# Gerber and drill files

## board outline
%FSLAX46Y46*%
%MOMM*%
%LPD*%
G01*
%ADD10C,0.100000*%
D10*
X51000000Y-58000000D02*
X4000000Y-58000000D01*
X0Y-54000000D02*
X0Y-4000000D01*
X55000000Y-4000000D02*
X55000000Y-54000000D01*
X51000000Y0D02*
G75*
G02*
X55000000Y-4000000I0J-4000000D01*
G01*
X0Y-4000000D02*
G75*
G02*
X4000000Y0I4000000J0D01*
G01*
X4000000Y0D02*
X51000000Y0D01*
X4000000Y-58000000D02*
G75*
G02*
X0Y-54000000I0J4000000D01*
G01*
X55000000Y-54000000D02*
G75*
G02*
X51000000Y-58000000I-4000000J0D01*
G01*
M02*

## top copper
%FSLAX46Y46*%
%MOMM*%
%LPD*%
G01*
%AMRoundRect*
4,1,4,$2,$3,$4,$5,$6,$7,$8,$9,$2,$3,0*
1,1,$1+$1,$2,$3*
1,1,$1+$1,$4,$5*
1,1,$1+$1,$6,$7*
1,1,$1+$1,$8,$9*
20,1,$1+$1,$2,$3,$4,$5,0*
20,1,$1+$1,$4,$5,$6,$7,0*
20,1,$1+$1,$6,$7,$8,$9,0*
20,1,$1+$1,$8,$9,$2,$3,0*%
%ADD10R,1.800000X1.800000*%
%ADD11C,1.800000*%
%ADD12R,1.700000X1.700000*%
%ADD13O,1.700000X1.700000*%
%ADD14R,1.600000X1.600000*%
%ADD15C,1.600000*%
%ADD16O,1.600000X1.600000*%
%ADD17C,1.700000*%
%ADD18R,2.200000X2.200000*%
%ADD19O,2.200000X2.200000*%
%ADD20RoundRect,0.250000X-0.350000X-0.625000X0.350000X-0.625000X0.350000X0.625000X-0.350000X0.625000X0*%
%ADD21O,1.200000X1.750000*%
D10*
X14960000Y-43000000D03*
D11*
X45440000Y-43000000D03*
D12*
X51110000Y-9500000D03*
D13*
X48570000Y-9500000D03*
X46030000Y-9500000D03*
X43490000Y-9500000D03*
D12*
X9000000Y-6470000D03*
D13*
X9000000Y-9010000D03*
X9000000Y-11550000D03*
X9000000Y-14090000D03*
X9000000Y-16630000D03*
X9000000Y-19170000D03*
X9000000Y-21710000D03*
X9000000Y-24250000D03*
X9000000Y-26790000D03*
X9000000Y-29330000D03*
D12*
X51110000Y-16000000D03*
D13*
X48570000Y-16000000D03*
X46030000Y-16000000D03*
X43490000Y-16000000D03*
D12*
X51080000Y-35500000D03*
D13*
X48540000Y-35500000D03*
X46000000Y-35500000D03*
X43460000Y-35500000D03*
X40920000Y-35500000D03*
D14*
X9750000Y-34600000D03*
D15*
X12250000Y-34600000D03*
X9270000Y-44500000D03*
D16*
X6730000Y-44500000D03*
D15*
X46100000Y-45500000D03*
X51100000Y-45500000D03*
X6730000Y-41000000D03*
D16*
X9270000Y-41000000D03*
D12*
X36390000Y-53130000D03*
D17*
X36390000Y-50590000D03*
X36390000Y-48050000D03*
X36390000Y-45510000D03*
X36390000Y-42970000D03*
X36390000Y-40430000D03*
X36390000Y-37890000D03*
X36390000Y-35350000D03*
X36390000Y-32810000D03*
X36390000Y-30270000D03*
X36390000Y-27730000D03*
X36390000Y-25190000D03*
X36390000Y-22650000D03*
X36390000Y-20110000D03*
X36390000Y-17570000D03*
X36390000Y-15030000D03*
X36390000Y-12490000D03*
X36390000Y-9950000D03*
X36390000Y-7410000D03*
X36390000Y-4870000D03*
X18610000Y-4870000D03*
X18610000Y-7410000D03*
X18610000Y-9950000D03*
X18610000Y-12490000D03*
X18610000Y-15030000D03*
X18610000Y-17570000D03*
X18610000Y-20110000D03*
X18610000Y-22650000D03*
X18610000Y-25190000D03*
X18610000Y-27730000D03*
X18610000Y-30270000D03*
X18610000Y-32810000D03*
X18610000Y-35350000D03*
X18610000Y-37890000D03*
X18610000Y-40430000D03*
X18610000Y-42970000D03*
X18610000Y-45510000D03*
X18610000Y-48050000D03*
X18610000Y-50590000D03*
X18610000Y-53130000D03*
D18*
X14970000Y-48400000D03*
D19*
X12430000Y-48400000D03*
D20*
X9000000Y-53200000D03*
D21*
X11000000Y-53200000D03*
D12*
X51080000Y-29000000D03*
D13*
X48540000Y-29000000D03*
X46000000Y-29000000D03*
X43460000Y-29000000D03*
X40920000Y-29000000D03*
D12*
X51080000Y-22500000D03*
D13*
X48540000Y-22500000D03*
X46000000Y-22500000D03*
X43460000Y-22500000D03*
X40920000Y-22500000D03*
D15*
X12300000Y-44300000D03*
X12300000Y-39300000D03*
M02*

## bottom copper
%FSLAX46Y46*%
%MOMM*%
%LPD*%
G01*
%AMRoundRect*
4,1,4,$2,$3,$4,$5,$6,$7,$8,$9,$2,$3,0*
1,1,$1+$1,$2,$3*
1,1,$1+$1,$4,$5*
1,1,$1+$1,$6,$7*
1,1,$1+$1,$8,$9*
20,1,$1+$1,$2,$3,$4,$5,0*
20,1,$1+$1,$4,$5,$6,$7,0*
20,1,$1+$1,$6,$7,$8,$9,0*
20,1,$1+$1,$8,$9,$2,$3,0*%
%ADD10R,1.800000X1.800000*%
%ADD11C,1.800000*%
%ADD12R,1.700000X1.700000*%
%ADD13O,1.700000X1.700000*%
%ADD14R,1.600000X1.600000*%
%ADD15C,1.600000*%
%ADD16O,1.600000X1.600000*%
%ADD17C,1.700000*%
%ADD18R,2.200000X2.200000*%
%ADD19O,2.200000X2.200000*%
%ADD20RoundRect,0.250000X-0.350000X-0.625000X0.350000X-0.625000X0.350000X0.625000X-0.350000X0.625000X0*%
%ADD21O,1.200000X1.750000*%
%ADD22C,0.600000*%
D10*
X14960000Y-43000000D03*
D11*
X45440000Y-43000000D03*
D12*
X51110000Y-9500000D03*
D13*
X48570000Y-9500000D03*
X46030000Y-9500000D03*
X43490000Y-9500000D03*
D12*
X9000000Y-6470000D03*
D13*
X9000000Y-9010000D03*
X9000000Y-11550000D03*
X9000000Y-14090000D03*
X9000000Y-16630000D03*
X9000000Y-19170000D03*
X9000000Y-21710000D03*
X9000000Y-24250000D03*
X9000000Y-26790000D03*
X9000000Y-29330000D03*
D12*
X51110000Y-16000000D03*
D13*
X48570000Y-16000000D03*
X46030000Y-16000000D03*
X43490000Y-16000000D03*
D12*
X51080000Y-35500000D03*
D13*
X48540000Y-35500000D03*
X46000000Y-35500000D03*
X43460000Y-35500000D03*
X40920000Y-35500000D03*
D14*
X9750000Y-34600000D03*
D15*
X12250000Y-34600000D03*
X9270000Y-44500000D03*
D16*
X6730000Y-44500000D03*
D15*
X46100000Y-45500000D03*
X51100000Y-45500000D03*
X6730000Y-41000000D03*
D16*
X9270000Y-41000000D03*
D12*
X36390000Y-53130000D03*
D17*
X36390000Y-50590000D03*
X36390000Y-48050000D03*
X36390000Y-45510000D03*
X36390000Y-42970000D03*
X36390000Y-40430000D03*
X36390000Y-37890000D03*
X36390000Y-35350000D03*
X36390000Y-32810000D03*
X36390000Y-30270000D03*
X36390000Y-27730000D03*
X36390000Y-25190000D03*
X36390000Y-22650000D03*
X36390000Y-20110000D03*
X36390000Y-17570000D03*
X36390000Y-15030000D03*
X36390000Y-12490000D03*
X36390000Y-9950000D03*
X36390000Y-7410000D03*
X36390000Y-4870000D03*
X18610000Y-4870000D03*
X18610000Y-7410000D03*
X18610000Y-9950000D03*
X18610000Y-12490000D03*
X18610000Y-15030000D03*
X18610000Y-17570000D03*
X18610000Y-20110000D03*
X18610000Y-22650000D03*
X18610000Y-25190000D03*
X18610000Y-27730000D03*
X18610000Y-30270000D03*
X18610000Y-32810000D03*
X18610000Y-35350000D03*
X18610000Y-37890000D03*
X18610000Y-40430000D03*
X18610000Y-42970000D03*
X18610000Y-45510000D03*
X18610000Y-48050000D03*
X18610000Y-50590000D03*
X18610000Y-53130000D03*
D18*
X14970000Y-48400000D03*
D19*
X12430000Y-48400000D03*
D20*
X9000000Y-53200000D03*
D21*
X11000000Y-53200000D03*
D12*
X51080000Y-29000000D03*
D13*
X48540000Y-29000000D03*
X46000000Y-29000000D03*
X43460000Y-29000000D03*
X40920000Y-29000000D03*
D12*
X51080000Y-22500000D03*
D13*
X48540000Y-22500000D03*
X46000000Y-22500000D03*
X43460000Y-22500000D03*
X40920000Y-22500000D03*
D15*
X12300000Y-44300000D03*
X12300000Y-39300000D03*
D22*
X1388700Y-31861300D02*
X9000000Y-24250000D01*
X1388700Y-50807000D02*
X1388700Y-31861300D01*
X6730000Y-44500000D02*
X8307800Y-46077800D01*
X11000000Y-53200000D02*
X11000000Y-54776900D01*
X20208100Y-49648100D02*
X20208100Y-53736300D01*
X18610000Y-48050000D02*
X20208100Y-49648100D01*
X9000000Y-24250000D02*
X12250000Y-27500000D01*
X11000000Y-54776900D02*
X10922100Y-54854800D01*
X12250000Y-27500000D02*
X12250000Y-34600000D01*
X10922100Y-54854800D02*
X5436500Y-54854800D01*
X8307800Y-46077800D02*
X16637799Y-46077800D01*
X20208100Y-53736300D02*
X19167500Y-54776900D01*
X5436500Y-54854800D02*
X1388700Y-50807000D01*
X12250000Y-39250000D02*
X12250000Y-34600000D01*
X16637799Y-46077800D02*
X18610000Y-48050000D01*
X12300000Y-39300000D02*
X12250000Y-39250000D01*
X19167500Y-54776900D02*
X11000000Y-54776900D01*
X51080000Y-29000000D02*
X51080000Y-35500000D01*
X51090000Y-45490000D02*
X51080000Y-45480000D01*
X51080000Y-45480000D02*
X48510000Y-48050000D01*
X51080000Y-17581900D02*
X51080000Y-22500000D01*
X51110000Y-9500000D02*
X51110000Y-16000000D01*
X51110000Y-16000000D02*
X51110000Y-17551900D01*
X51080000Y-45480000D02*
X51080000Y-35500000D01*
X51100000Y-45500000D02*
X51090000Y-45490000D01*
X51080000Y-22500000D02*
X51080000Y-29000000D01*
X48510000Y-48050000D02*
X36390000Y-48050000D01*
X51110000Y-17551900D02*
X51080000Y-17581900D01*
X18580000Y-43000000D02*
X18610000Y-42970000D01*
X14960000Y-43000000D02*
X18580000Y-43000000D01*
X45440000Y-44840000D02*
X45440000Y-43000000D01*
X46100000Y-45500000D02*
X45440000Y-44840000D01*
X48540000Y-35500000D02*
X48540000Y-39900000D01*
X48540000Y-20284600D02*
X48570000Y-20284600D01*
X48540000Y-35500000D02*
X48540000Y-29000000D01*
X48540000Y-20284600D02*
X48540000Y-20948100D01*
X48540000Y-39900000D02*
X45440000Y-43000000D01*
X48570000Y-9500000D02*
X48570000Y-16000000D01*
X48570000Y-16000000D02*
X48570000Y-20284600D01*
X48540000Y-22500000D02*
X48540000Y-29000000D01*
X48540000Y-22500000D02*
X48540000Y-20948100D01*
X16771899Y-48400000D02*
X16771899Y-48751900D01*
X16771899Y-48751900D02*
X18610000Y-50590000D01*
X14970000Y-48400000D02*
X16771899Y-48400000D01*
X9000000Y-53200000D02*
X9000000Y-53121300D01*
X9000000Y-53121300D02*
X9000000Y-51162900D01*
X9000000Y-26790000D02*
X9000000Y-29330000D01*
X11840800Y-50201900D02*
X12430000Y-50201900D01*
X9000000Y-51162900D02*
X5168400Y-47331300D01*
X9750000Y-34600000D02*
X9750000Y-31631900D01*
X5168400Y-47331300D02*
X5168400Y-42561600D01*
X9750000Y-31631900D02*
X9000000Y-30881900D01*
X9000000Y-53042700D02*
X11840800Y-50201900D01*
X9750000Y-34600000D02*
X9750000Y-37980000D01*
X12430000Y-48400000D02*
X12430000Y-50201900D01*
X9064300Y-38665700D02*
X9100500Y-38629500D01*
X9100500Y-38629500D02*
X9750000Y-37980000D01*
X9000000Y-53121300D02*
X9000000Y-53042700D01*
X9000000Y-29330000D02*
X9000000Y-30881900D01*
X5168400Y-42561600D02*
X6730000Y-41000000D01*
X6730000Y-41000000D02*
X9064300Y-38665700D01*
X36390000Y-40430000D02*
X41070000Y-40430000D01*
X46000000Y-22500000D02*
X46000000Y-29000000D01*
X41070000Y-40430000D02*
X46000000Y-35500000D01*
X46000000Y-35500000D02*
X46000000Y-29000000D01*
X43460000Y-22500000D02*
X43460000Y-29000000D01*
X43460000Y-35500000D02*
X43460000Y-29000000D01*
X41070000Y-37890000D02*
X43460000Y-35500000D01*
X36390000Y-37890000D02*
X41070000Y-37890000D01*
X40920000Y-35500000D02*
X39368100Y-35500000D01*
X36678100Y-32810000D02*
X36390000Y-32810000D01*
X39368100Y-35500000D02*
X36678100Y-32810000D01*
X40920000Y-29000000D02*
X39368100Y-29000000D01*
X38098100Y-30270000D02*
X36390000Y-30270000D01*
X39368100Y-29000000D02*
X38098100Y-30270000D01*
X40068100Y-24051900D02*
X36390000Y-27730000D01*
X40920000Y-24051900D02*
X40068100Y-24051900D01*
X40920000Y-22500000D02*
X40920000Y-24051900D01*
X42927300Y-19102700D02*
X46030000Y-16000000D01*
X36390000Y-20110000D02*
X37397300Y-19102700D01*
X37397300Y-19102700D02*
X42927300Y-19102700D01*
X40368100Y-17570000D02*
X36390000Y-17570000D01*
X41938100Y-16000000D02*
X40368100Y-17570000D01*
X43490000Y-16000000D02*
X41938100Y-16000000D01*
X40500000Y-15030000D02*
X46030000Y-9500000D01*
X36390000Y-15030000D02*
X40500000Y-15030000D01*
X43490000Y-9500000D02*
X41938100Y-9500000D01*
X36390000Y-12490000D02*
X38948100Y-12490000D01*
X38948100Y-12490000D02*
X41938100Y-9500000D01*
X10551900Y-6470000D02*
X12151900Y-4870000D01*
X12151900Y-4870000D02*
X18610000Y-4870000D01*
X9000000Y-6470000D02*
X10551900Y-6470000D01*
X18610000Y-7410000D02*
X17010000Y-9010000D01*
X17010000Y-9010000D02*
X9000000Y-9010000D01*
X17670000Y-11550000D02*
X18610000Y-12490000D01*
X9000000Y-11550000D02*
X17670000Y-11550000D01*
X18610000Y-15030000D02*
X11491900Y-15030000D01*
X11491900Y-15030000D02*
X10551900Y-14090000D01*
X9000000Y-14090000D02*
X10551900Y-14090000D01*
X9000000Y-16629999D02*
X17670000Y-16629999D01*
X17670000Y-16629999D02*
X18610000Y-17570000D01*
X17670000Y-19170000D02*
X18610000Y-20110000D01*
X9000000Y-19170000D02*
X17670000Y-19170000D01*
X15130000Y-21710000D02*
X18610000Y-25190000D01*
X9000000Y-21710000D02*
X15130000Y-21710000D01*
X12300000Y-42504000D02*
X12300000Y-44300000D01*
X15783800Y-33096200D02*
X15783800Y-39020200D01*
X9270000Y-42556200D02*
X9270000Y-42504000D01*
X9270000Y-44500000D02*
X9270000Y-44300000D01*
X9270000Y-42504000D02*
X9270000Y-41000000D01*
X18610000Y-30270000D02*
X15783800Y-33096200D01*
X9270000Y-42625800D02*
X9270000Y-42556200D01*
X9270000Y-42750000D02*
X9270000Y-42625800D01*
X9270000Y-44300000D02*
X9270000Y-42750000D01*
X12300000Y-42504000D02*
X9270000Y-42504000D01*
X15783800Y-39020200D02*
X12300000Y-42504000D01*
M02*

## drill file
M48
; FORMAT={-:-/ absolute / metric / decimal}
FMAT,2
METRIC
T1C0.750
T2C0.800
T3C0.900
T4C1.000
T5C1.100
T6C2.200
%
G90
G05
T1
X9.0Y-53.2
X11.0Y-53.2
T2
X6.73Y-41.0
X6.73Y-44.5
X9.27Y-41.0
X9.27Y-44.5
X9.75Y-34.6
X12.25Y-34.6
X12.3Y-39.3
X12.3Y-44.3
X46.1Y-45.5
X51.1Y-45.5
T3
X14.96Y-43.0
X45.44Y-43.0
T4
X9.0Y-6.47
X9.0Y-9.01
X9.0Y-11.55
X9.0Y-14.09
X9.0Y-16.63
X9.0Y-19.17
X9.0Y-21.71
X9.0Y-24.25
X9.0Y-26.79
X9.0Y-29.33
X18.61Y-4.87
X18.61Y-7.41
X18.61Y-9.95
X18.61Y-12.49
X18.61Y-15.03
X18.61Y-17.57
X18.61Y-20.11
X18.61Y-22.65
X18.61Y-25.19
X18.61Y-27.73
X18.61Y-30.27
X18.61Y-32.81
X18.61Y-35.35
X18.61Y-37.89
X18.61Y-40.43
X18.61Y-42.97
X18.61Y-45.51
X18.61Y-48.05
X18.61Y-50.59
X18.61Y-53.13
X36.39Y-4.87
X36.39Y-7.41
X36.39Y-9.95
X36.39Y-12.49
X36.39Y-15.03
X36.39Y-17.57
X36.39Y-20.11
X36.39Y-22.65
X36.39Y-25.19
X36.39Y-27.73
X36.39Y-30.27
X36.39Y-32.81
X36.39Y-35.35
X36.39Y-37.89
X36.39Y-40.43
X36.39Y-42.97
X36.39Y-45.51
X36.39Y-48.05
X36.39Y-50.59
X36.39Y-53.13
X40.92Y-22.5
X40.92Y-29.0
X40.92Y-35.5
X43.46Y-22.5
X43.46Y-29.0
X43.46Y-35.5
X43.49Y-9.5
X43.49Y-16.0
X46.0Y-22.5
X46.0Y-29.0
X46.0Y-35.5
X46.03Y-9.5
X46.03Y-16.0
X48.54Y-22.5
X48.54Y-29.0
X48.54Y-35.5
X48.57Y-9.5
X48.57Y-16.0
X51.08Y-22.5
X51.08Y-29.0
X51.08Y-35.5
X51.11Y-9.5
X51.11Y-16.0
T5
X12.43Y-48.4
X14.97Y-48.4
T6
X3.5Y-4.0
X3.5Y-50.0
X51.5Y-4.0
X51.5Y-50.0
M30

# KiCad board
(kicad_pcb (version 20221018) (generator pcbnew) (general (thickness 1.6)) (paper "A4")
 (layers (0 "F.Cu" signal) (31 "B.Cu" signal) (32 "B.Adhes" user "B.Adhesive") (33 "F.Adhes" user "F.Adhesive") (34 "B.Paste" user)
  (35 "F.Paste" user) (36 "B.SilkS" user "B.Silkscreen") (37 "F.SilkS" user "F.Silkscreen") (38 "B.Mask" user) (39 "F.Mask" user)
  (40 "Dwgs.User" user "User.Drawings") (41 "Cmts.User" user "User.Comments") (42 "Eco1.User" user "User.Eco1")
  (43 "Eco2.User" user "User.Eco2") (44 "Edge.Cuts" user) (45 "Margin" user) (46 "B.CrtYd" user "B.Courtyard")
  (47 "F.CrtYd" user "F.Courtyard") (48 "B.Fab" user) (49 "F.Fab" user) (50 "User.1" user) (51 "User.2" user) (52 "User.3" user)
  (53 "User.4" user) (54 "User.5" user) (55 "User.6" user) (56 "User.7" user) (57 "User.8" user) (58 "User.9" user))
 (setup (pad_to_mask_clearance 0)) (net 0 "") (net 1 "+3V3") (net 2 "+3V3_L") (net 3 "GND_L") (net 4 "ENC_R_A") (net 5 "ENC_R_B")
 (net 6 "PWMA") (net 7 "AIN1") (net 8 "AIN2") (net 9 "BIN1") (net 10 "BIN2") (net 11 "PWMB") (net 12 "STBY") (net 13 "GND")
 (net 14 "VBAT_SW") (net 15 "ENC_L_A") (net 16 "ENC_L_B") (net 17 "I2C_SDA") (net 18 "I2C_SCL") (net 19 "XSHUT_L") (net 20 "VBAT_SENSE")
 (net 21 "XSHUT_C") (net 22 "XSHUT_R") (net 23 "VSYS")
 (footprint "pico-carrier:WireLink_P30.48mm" (layer "F.Cu") (at 30.2 43)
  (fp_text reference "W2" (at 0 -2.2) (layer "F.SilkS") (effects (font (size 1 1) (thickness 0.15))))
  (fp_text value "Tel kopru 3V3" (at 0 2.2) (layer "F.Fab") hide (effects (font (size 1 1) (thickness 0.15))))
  (pad "1" thru_hole rect (at -15.24 0) (size 1.8 1.8) (drill 0.9) (layers "*.Cu" "*.Mask") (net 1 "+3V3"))
  (pad "2" thru_hole circle (at 15.24 0) (size 1.8 1.8) (drill 0.9) (layers "*.Cu" "*.Mask") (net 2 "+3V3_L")))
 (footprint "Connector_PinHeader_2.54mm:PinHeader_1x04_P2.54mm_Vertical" (layer "F.Cu") (at 51.11 9.5 -90)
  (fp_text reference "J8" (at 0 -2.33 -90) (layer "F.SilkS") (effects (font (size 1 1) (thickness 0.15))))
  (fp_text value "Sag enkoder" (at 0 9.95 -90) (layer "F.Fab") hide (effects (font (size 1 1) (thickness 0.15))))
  (pad "1" thru_hole rect (at 0 0 270) (size 1.7 1.7) (drill 1) (layers "*.Cu" "*.Mask") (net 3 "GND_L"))
  (pad "2" thru_hole oval (at 0 2.54 270) (size 1.7 1.7) (drill 1) (layers "*.Cu" "*.Mask") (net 2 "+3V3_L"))
  (pad "3" thru_hole oval (at 0 5.08 270) (size 1.7 1.7) (drill 1) (layers "*.Cu" "*.Mask") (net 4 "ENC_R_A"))
  (pad "4" thru_hole oval (at 0 7.62 270) (size 1.7 1.7) (drill 1) (layers "*.Cu" "*.Mask") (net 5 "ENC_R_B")))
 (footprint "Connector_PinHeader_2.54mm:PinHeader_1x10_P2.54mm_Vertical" (layer "F.Cu") (at 9 6.47)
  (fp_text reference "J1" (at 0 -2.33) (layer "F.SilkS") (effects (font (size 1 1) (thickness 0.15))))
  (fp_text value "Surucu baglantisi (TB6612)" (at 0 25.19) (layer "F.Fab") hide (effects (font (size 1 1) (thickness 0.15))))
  (pad "1" thru_hole rect (at 0 0) (size 1.7 1.7) (drill 1) (layers "*.Cu" "*.Mask") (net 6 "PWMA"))
  (pad "2" thru_hole oval (at 0 2.54) (size 1.7 1.7) (drill 1) (layers "*.Cu" "*.Mask") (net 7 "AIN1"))
  (pad "3" thru_hole oval (at 0 5.08) (size 1.7 1.7) (drill 1) (layers "*.Cu" "*.Mask") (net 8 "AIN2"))
  (pad "4" thru_hole oval (at 0 7.62) (size 1.7 1.7) (drill 1) (layers "*.Cu" "*.Mask") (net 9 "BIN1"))
  (pad "5" thru_hole oval (at 0 10.16) (size 1.7 1.7) (drill 1) (layers "*.Cu" "*.Mask") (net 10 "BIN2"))
  (pad "6" thru_hole oval (at 0 12.7) (size 1.7 1.7) (drill 1) (layers "*.Cu" "*.Mask") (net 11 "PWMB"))
  (pad "7" thru_hole oval (at 0 15.24) (size 1.7 1.7) (drill 1) (layers "*.Cu" "*.Mask") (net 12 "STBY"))
  (pad "8" thru_hole oval (at 0 17.78) (size 1.7 1.7) (drill 1) (layers "*.Cu" "*.Mask") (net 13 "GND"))
  (pad "9" thru_hole oval (at 0 20.32) (size 1.7 1.7) (drill 1) (layers "*.Cu" "*.Mask") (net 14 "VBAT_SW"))
  (pad "10" thru_hole oval (at 0 22.86) (size 1.7 1.7) (drill 1) (layers "*.Cu" "*.Mask") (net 14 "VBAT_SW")))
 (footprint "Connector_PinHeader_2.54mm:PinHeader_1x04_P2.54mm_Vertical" (layer "F.Cu") (at 51.11 16 -90)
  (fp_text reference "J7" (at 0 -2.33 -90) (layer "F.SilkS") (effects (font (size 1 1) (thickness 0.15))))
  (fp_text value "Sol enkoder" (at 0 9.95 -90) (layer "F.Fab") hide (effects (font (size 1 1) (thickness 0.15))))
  (pad "1" thru_hole rect (at 0 0 270) (size 1.7 1.7) (drill 1) (layers "*.Cu" "*.Mask") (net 3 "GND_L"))
  (pad "2" thru_hole oval (at 0 2.54 270) (size 1.7 1.7) (drill 1) (layers "*.Cu" "*.Mask") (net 2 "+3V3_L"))
  (pad "3" thru_hole oval (at 0 5.08 270) (size 1.7 1.7) (drill 1) (layers "*.Cu" "*.Mask") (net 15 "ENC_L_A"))
  (pad "4" thru_hole oval (at 0 7.62 270) (size 1.7 1.7) (drill 1) (layers "*.Cu" "*.Mask") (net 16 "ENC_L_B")))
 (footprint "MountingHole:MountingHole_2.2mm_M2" (layer "F.Cu") (at 51.5 50)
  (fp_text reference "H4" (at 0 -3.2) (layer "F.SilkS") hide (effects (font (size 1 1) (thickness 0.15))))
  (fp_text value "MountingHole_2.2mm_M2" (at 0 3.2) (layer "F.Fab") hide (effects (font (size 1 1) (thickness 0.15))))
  (pad "" np_thru_hole circle (at 0 0) (size 2.2 2.2) (drill 2.2) (layers "*.Cu" "*.Mask")))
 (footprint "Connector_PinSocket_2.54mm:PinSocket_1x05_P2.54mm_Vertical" (layer "F.Cu") (at 51.08 35.5 -90)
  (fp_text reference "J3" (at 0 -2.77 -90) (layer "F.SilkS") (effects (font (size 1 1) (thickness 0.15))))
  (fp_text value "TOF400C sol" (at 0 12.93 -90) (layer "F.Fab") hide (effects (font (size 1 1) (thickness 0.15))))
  (pad "1" thru_hole rect (at 0 0 270) (size 1.7 1.7) (drill 1) (layers "*.Cu" "*.Mask") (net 3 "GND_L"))
  (pad "2" thru_hole oval (at 0 2.54 270) (size 1.7 1.7) (drill 1) (layers "*.Cu" "*.Mask") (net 2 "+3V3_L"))
  (pad "3" thru_hole oval (at 0 5.08 270) (size 1.7 1.7) (drill 1) (layers "*.Cu" "*.Mask") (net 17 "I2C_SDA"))
  (pad "4" thru_hole oval (at 0 7.62 270) (size 1.7 1.7) (drill 1) (layers "*.Cu" "*.Mask") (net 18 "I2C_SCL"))
  (pad "5" thru_hole oval (at 0 10.16 270) (size 1.7 1.7) (drill 1) (layers "*.Cu" "*.Mask") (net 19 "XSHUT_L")))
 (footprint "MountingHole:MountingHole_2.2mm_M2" (layer "F.Cu") (at 51.5 4)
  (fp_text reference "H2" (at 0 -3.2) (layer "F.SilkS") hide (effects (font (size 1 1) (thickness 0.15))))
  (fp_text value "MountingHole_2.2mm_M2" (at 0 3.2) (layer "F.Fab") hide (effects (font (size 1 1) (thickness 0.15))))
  (pad "" np_thru_hole circle (at 0 0) (size 2.2 2.2) (drill 2.2) (layers "*.Cu" "*.Mask")))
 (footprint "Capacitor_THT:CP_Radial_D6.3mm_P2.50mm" (layer "F.Cu") (at 9.75 34.6)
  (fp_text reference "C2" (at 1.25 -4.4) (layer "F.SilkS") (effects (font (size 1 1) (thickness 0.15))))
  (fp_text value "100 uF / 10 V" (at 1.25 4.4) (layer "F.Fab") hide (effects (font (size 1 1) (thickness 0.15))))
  (pad "1" thru_hole rect (at 0 0) (size 1.6 1.6) (drill 0.8) (layers "*.Cu" "*.Mask") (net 14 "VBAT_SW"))
  (pad "2" thru_hole circle (at 2.5 0) (size 1.6 1.6) (drill 0.8) (layers "*.Cu" "*.Mask") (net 13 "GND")))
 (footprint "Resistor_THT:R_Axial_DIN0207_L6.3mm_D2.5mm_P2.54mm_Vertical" (layer "F.Cu") (at 9.27 44.5 180)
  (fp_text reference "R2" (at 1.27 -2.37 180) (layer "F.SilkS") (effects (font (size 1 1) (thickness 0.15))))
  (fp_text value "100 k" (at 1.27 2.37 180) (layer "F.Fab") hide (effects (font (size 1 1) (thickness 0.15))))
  (pad "1" thru_hole circle (at 0 0 180) (size 1.6 1.6) (drill 0.8) (layers "*.Cu" "*.Mask") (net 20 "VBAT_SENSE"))
  (pad "2" thru_hole oval (at 2.54 0 180) (size 1.6 1.6) (drill 0.8) (layers "*.Cu" "*.Mask") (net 13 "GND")))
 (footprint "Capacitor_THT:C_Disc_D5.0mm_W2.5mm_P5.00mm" (layer "F.Cu") (at 46.1 45.5)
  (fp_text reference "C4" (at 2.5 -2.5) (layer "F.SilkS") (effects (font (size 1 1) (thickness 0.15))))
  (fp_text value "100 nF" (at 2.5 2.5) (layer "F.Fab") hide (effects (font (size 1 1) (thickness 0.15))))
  (pad "1" thru_hole circle (at 0 0) (size 1.6 1.6) (drill 0.8) (layers "*.Cu" "*.Mask") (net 2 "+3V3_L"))
  (pad "2" thru_hole circle (at 5 0) (size 1.6 1.6) (drill 0.8) (layers "*.Cu" "*.Mask") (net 3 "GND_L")))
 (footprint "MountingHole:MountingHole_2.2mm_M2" (layer "F.Cu") (at 3.5 4)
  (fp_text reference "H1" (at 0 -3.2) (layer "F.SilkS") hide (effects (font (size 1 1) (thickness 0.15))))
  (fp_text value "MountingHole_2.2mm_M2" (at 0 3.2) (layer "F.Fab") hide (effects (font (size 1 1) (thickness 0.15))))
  (pad "" np_thru_hole circle (at 0 0) (size 2.2 2.2) (drill 2.2) (layers "*.Cu" "*.Mask")))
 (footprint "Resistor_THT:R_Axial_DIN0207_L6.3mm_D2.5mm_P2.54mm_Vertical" (layer "F.Cu") (at 6.73 41)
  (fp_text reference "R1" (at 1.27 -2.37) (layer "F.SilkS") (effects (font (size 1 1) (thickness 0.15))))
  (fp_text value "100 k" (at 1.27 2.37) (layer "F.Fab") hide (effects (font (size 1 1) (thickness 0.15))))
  (pad "1" thru_hole circle (at 0 0) (size 1.6 1.6) (drill 0.8) (layers "*.Cu" "*.Mask") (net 14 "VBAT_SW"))
  (pad "2" thru_hole oval (at 2.54 0) (size 1.6 1.6) (drill 0.8) (layers "*.Cu" "*.Mask") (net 20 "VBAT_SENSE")))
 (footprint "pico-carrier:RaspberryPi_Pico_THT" (layer "F.Cu") (at 36.39 53.13 180)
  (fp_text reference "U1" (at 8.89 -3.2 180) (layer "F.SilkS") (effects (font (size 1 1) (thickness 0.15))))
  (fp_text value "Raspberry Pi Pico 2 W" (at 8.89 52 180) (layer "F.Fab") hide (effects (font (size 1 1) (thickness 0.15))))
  (pad "1" thru_hole rect (at 0 0 180) (size 1.7 1.7) (drill 1) (layers "*.Cu" "*.Mask"))
  (pad "2" thru_hole circle (at 0 2.54 180) (size 1.7 1.7) (drill 1) (layers "*.Cu" "*.Mask"))
  (pad "3" thru_hole circle (at 0 5.08 180) (size 1.7 1.7) (drill 1) (layers "*.Cu" "*.Mask") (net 3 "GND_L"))
  (pad "4" thru_hole circle (at 0 7.62 180) (size 1.7 1.7) (drill 1) (layers "*.Cu" "*.Mask"))
  (pad "5" thru_hole circle (at 0 10.16 180) (size 1.7 1.7) (drill 1) (layers "*.Cu" "*.Mask"))
  (pad "6" thru_hole circle (at 0 12.7 180) (size 1.7 1.7) (drill 1) (layers "*.Cu" "*.Mask") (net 17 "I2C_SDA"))
  (pad "7" thru_hole circle (at 0 15.24 180) (size 1.7 1.7) (drill 1) (layers "*.Cu" "*.Mask") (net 18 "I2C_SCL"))
  (pad "8" thru_hole circle (at 0 17.78 180) (size 1.7 1.7) (drill 1) (layers "*.Cu" "*.Mask"))
  (pad "9" thru_hole circle (at 0 20.32 180) (size 1.7 1.7) (drill 1) (layers "*.Cu" "*.Mask") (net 19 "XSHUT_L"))
  (pad "10" thru_hole circle (at 0 22.86 180) (size 1.7 1.7) (drill 1) (layers "*.Cu" "*.Mask") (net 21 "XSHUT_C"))
  (pad "11" thru_hole circle (at 0 25.4 180) (size 1.7 1.7) (drill 1) (layers "*.Cu" "*.Mask") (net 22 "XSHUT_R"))
  (pad "12" thru_hole circle (at 0 27.94 180) (size 1.7 1.7) (drill 1) (layers "*.Cu" "*.Mask"))
  (pad "13" thru_hole circle (at 0 30.48 180) (size 1.7 1.7) (drill 1) (layers "*.Cu" "*.Mask"))
  (pad "14" thru_hole circle (at 0 33.02 180) (size 1.7 1.7) (drill 1) (layers "*.Cu" "*.Mask") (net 15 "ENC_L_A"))
  (pad "15" thru_hole circle (at 0 35.56 180) (size 1.7 1.7) (drill 1) (layers "*.Cu" "*.Mask") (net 16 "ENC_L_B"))
  (pad "16" thru_hole circle (at 0 38.1 180) (size 1.7 1.7) (drill 1) (layers "*.Cu" "*.Mask") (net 4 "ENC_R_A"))
  (pad "17" thru_hole circle (at 0 40.64 180) (size 1.7 1.7) (drill 1) (layers "*.Cu" "*.Mask") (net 5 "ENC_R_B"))
  (pad "18" thru_hole circle (at 0 43.18 180) (size 1.7 1.7) (drill 1) (layers "*.Cu" "*.Mask"))
  (pad "19" thru_hole circle (at 0 45.72 180) (size 1.7 1.7) (drill 1) (layers "*.Cu" "*.Mask"))
  (pad "20" thru_hole circle (at 0 48.26 180) (size 1.7 1.7) (drill 1) (layers "*.Cu" "*.Mask"))
  (pad "21" thru_hole circle (at 17.78 48.26 180) (size 1.7 1.7) (drill 1) (layers "*.Cu" "*.Mask") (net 6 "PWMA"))
  (pad "22" thru_hole circle (at 17.78 45.72 180) (size 1.7 1.7) (drill 1) (layers "*.Cu" "*.Mask") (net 7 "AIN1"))
  (pad "23" thru_hole circle (at 17.78 43.18 180) (size 1.7 1.7) (drill 1) (layers "*.Cu" "*.Mask"))
  (pad "24" thru_hole circle (at 17.78 40.64 180) (size 1.7 1.7) (drill 1) (layers "*.Cu" "*.Mask") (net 8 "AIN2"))
  (pad "25" thru_hole circle (at 17.78 38.1 180) (size 1.7 1.7) (drill 1) (layers "*.Cu" "*.Mask") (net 9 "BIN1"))
  (pad "26" thru_hole circle (at 17.78 35.56 180) (size 1.7 1.7) (drill 1) (layers "*.Cu" "*.Mask") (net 10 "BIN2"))
  (pad "27" thru_hole circle (at 17.78 33.02 180) (size 1.7 1.7) (drill 1) (layers "*.Cu" "*.Mask") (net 11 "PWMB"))
  (pad "28" thru_hole circle (at 17.78 30.48 180) (size 1.7 1.7) (drill 1) (layers "*.Cu" "*.Mask"))
  (pad "29" thru_hole circle (at 17.78 27.94 180) (size 1.7 1.7) (drill 1) (layers "*.Cu" "*.Mask") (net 12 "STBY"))
  (pad "30" thru_hole circle (at 17.78 25.4 180) (size 1.7 1.7) (drill 1) (layers "*.Cu" "*.Mask"))
  (pad "31" thru_hole circle (at 17.78 22.86 180) (size 1.7 1.7) (drill 1) (layers "*.Cu" "*.Mask") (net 20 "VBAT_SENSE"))
  (pad "32" thru_hole circle (at 17.78 20.32 180) (size 1.7 1.7) (drill 1) (layers "*.Cu" "*.Mask"))
  (pad "33" thru_hole circle (at 17.78 17.78 180) (size 1.7 1.7) (drill 1) (layers "*.Cu" "*.Mask"))
  (pad "34" thru_hole circle (at 17.78 15.24 180) (size 1.7 1.7) (drill 1) (layers "*.Cu" "*.Mask"))
  (pad "35" thru_hole circle (at 17.78 12.7 180) (size 1.7 1.7) (drill 1) (layers "*.Cu" "*.Mask"))
  (pad "36" thru_hole circle (at 17.78 10.16 180) (size 1.7 1.7) (drill 1) (layers "*.Cu" "*.Mask") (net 1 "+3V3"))
  (pad "37" thru_hole circle (at 17.78 7.62 180) (size 1.7 1.7) (drill 1) (layers "*.Cu" "*.Mask"))
  (pad "38" thru_hole circle (at 17.78 5.08 180) (size 1.7 1.7) (drill 1) (layers "*.Cu" "*.Mask") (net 13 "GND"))
  (pad "39" thru_hole circle (at 17.78 2.54 180) (size 1.7 1.7) (drill 1) (layers "*.Cu" "*.Mask") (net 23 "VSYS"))
  (pad "40" thru_hole circle (at 17.78 0 180) (size 1.7 1.7) (drill 1) (layers "*.Cu" "*.Mask")))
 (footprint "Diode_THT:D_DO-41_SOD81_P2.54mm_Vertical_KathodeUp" (layer "F.Cu") (at 14.97 48.4 180)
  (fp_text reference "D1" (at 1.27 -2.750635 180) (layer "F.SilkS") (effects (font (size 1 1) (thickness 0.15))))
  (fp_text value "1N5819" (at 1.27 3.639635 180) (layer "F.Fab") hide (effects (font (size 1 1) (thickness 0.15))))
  (pad "1" thru_hole rect (at 0 0 180) (size 2.2 2.2) (drill 1.1) (layers "*.Cu" "*.Mask") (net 23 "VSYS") (clearance 0.3))
  (pad "2" thru_hole oval (at 2.54 0 180) (size 2.2 2.2) (drill 1.1) (layers "*.Cu" "*.Mask") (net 14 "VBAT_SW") (clearance 0.3)))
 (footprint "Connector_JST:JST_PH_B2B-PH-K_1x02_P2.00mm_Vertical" (layer "F.Cu") (at 9 53.2)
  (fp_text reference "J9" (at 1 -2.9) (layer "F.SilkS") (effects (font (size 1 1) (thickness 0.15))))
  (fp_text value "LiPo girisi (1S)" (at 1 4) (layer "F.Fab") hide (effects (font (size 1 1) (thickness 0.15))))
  (pad "1" thru_hole roundrect (at 0 0) (size 1.2 1.75) (drill 0.75) (layers "*.Cu" "*.Mask") (roundrect_rratio 0.208333) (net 14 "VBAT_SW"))
  (pad "2" thru_hole oval (at 2 0) (size 1.2 1.75) (drill 0.75) (layers "*.Cu" "*.Mask") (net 13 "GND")))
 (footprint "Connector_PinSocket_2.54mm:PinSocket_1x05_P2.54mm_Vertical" (layer "F.Cu") (at 51.08 29 -90)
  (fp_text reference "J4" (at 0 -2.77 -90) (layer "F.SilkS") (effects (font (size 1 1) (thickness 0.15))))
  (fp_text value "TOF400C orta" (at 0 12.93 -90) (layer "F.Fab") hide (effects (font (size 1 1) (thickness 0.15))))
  (pad "1" thru_hole rect (at 0 0 270) (size 1.7 1.7) (drill 1) (layers "*.Cu" "*.Mask") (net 3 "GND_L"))
  (pad "2" thru_hole oval (at 0 2.54 270) (size 1.7 1.7) (drill 1) (layers "*.Cu" "*.Mask") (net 2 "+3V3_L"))
  (pad "3" thru_hole oval (at 0 5.08 270) (size 1.7 1.7) (drill 1) (layers "*.Cu" "*.Mask") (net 17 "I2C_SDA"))
  (pad "4" thru_hole oval (at 0 7.62 270) (size 1.7 1.7) (drill 1) (layers "*.Cu" "*.Mask") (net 18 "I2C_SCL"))
  (pad "5" thru_hole oval (at 0 10.16 270) (size 1.7 1.7) (drill 1) (layers "*.Cu" "*.Mask") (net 21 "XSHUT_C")))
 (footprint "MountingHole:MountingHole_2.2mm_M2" (layer "F.Cu") (at 3.5 50)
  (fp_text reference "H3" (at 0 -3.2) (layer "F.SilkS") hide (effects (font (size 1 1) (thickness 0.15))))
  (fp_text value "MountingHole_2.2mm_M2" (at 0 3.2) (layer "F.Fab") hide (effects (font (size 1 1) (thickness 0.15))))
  (pad "" np_thru_hole circle (at 0 0) (size 2.2 2.2) (drill 2.2) (layers "*.Cu" "*.Mask")))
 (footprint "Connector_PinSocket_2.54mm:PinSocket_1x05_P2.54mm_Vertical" (layer "F.Cu") (at 51.08 22.5 -90)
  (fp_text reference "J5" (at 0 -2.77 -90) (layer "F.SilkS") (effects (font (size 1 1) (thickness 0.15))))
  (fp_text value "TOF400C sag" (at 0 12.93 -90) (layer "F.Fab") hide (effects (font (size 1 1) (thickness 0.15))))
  (pad "1" thru_hole rect (at 0 0 270) (size 1.7 1.7) (drill 1) (layers "*.Cu" "*.Mask") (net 3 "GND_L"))
  (pad "2" thru_hole oval (at 0 2.54 270) (size 1.7 1.7) (drill 1) (layers "*.Cu" "*.Mask") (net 2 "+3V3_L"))
  (pad "3" thru_hole oval (at 0 5.08 270) (size 1.7 1.7) (drill 1) (layers "*.Cu" "*.Mask") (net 17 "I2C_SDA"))
  (pad "4" thru_hole oval (at 0 7.62 270) (size 1.7 1.7) (drill 1) (layers "*.Cu" "*.Mask") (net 18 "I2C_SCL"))
  (pad "5" thru_hole oval (at 0 10.16 270) (size 1.7 1.7) (drill 1) (layers "*.Cu" "*.Mask") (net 22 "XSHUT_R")))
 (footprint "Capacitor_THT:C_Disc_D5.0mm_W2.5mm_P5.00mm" (layer "F.Cu") (at 12.3 44.3 90)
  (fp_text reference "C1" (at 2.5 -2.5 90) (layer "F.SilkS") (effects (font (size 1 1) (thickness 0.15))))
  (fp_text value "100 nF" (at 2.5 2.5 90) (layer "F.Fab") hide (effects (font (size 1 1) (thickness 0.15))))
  (pad "1" thru_hole circle (at 0 0 90) (size 1.6 1.6) (drill 0.8) (layers "*.Cu" "*.Mask") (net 20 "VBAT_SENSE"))
  (pad "2" thru_hole circle (at 5 0 90) (size 1.6 1.6) (drill 0.8) (layers "*.Cu" "*.Mask") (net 13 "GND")))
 (gr_line (start 51 58) (end 4 58) (stroke (width 0.1) (type default)) (layer "Edge.Cuts"))
 (gr_line (start 0 54) (end 0 4) (stroke (width 0.1) (type default)) (layer "Edge.Cuts"))
 (gr_line (start 55 4) (end 55 54) (stroke (width 0.1) (type default)) (layer "Edge.Cuts"))
 (gr_arc (start 51 0) (mid 53.828427 1.171573) (end 55 4) (stroke (width 0.1) (type default)) (layer "Edge.Cuts"))
 (gr_arc (start 0 4) (mid 1.171573 1.171573) (end 4 0) (stroke (width 0.1) (type default)) (layer "Edge.Cuts"))
 (gr_line (start 4 0) (end 51 0) (stroke (width 0.1) (type default)) (layer "Edge.Cuts"))
 (gr_arc (start 4 58) (mid 1.171573 56.828427) (end 0 54) (stroke (width 0.1) (type default)) (layer "Edge.Cuts"))
 (gr_arc (start 55 54) (mid 53.828427 56.828427) (end 51 58) (stroke (width 0.1) (type default)) (layer "Edge.Cuts"))
 (segment (start 1.3887 31.8613) (end 9 24.25) (width 0.6) (layer "B.Cu") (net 13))
 (segment (start 1.3887 50.807) (end 1.3887 31.8613) (width 0.6) (layer "B.Cu") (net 13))
 (segment (start 6.73 44.5) (end 8.3078 46.0778) (width 0.6) (layer "B.Cu") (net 13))
 (segment (start 11 53.2) (end 11 54.7769) (width 0.6) (layer "B.Cu") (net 13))
 (segment (start 20.2081 49.6481) (end 20.2081 53.7363) (width 0.6) (layer "B.Cu") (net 13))
 (segment (start 18.61 48.05) (end 20.2081 49.6481) (width 0.6) (layer "B.Cu") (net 13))
 (segment (start 9 24.25) (end 12.25 27.5) (width 0.6) (layer "B.Cu") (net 13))
 (segment (start 11 54.7769) (end 10.9221 54.8548) (width 0.6) (layer "B.Cu") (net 13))
 (segment (start 12.25 27.5) (end 12.25 34.6) (width 0.6) (layer "B.Cu") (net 13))
 (segment (start 10.9221 54.8548) (end 5.4365 54.8548) (width 0.6) (layer "B.Cu") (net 13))
 (segment (start 8.3078 46.0778) (end 16.637799 46.0778) (width 0.6) (layer "B.Cu") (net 13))
 (segment (start 20.2081 53.7363) (end 19.1675 54.7769) (width 0.6) (layer "B.Cu") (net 13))
 (segment (start 5.4365 54.8548) (end 1.3887 50.807) (width 0.6) (layer "B.Cu") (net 13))
 (segment (start 12.25 39.25) (end 12.25 34.6) (width 0.6) (layer "B.Cu") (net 13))
 (segment (start 16.637799 46.0778) (end 18.61 48.05) (width 0.6) (layer "B.Cu") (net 13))
 (segment (start 12.3 39.3) (end 12.25 39.25) (width 0.6) (layer "B.Cu") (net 13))
 (segment (start 19.1675 54.7769) (end 11 54.7769) (width 0.6) (layer "B.Cu") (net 13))
 (segment (start 51.08 29) (end 51.08 35.5) (width 0.6) (layer "B.Cu") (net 3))
 (segment (start 51.09 45.49) (end 51.08 45.48) (width 0.6) (layer "B.Cu") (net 3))
 (segment (start 51.08 45.48) (end 48.51 48.05) (width 0.6) (layer "B.Cu") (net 3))
 (segment (start 51.08 17.5819) (end 51.08 22.5) (width 0.6) (layer "B.Cu") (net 3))
 (segment (start 51.11 9.5) (end 51.11 16) (width 0.6) (layer "B.Cu") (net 3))
 (segment (start 51.11 16) (end 51.11 17.5519) (width 0.6) (layer "B.Cu") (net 3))
 (segment (start 51.08 45.48) (end 51.08 35.5) (width 0.6) (layer "B.Cu") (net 3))
 (segment (start 51.1 45.5) (end 51.09 45.49) (width 0.6) (layer "B.Cu") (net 3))
 (segment (start 51.08 22.5) (end 51.08 29) (width 0.6) (layer "B.Cu") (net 3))
 (segment (start 48.51 48.05) (end 36.39 48.05) (width 0.6) (layer "B.Cu") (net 3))
 (segment (start 51.11 17.5519) (end 51.08 17.5819) (width 0.6) (layer "B.Cu") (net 3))
 (segment (start 18.58 43) (end 18.61 42.97) (width 0.6) (layer "B.Cu") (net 1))
 (segment (start 14.96 43) (end 18.58 43) (width 0.6) (layer "B.Cu") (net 1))
 (segment (start 45.44 44.84) (end 45.44 43) (width 0.6) (layer "B.Cu") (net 2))
 (segment (start 46.1 45.5) (end 45.44 44.84) (width 0.6) (layer "B.Cu") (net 2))
 (segment (start 48.54 35.5) (end 48.54 39.9) (width 0.6) (layer "B.Cu") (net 2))
 (segment (start 48.54 20.2846) (end 48.57 20.2846) (width 0.6) (layer "B.Cu") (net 2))
 (segment (start 48.54 35.5) (end 48.54 29) (width 0.6) (layer "B.Cu") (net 2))
 (segment (start 48.54 20.2846) (end 48.54 20.9481) (width 0.6) (layer "B.Cu") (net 2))
 (segment (start 48.54 39.9) (end 45.44 43) (width 0.6) (layer "B.Cu") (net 2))
 (segment (start 48.57 9.5) (end 48.57 16) (width 0.6) (layer "B.Cu") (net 2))
 (segment (start 48.57 16) (end 48.57 20.2846) (width 0.6) (layer "B.Cu") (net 2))
 (segment (start 48.54 22.5) (end 48.54 29) (width 0.6) (layer "B.Cu") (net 2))
 (segment (start 48.54 22.5) (end 48.54 20.9481) (width 0.6) (layer "B.Cu") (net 2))
 (segment (start 16.771899 48.4) (end 16.771899 48.7519) (width 0.6) (layer "B.Cu") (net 23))
 (segment (start 16.771899 48.7519) (end 18.61 50.59) (width 0.6) (layer "B.Cu") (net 23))
 (segment (start 14.97 48.4) (end 16.771899 48.4) (width 0.6) (layer "B.Cu") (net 23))
 (segment (start 9 53.2) (end 9 53.1213) (width 0.6) (layer "B.Cu") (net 14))
 (segment (start 9 53.1213) (end 9 51.1629) (width 0.6) (layer "B.Cu") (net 14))
 (segment (start 9 26.79) (end 9 29.33) (width 0.6) (layer "B.Cu") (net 14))
 (segment (start 11.8408 50.2019) (end 12.43 50.2019) (width 0.6) (layer "B.Cu") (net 14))
 (segment (start 9 51.1629) (end 5.1684 47.3313) (width 0.6) (layer "B.Cu") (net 14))
 (segment (start 9.75 34.6) (end 9.75 31.6319) (width 0.6) (layer "B.Cu") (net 14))
 (segment (start 5.1684 47.3313) (end 5.1684 42.5616) (width 0.6) (layer "B.Cu") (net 14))
 (segment (start 9.75 31.6319) (end 9 30.8819) (width 0.6) (layer "B.Cu") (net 14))
 (segment (start 9 53.0427) (end 11.8408 50.2019) (width 0.6) (layer "B.Cu") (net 14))
 (segment (start 9.75 34.6) (end 9.75 37.98) (width 0.6) (layer "B.Cu") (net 14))
 (segment (start 12.43 48.4) (end 12.43 50.2019) (width 0.6) (layer "B.Cu") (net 14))
 (segment (start 9.0643 38.6657) (end 9.1005 38.6295) (width 0.6) (layer "B.Cu") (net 14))
 (segment (start 9.1005 38.6295) (end 9.75 37.98) (width 0.6) (layer "B.Cu") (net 14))
 (segment (start 9 53.1213) (end 9 53.0427) (width 0.6) (layer "B.Cu") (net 14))
 (segment (start 9 29.33) (end 9 30.8819) (width 0.6) (layer "B.Cu") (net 14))
 (segment (start 5.1684 42.5616) (end 6.73 41) (width 0.6) (layer "B.Cu") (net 14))
 (segment (start 6.73 41) (end 9.0643 38.6657) (width 0.6) (layer "B.Cu") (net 14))
 (segment (start 36.39 40.43) (end 41.07 40.43) (width 0.6) (layer "B.Cu") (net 17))
 (segment (start 46 22.5) (end 46 29) (width 0.6) (layer "B.Cu") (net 17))
 (segment (start 41.07 40.43) (end 46 35.5) (width 0.6) (layer "B.Cu") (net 17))
 (segment (start 46 35.5) (end 46 29) (width 0.6) (layer "B.Cu") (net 17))
 (segment (start 43.46 22.5) (end 43.46 29) (width 0.6) (layer "B.Cu") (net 18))
 (segment (start 43.46 35.5) (end 43.46 29) (width 0.6) (layer "B.Cu") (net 18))
 (segment (start 41.07 37.89) (end 43.46 35.5) (width 0.6) (layer "B.Cu") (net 18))
 (segment (start 36.39 37.89) (end 41.07 37.89) (width 0.6) (layer "B.Cu") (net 18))
 (segment (start 40.92 35.5) (end 39.3681 35.5) (width 0.6) (layer "B.Cu") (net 19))
 (segment (start 36.6781 32.81) (end 36.39 32.81) (width 0.6) (layer "B.Cu") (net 19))
 (segment (start 39.3681 35.5) (end 36.6781 32.81) (width 0.6) (layer "B.Cu") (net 19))
 (segment (start 40.92 29) (end 39.3681 29) (width 0.6) (layer "B.Cu") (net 21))
 (segment (start 38.0981 30.27) (end 36.39 30.27) (width 0.6) (layer "B.Cu") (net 21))
 (segment (start 39.3681 29) (end 38.0981 30.27) (width 0.6) (layer "B.Cu") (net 21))
 (segment (start 40.0681 24.0519) (end 36.39 27.73) (width 0.6) (layer "B.Cu") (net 22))
 (segment (start 40.92 24.0519) (end 40.0681 24.0519) (width 0.6) (layer "B.Cu") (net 22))
 (segment (start 40.92 22.5) (end 40.92 24.0519) (width 0.6) (layer "B.Cu") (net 22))
 (segment (start 42.9273 19.1027) (end 46.03 16) (width 0.6) (layer "B.Cu") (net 15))
 (segment (start 36.39 20.11) (end 37.3973 19.1027) (width 0.6) (layer "B.Cu") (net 15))
 (segment (start 37.3973 19.1027) (end 42.9273 19.1027) (width 0.6) (layer "B.Cu") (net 15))
 (segment (start 40.3681 17.57) (end 36.39 17.57) (width 0.6) (layer "B.Cu") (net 16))
 (segment (start 41.9381 16) (end 40.3681 17.57) (width 0.6) (layer "B.Cu") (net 16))
 (segment (start 43.49 16) (end 41.9381 16) (width 0.6) (layer "B.Cu") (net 16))
 (segment (start 40.5 15.03) (end 46.03 9.5) (width 0.6) (layer "B.Cu") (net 4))
 (segment (start 36.39 15.03) (end 40.5 15.03) (width 0.6) (layer "B.Cu") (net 4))
 (segment (start 43.49 9.5) (end 41.9381 9.5) (width 0.6) (layer "B.Cu") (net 5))
 (segment (start 36.39 12.49) (end 38.9481 12.49) (width 0.6) (layer "B.Cu") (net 5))
 (segment (start 38.9481 12.49) (end 41.9381 9.5) (width 0.6) (layer "B.Cu") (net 5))
 (segment (start 10.5519 6.47) (end 12.1519 4.87) (width 0.6) (layer "B.Cu") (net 6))
 (segment (start 12.1519 4.87) (end 18.61 4.87) (width 0.6) (layer "B.Cu") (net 6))
 (segment (start 9 6.47) (end 10.5519 6.47) (width 0.6) (layer "B.Cu") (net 6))
 (segment (start 18.61 7.41) (end 17.01 9.01) (width 0.6) (layer "B.Cu") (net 7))
 (segment (start 17.01 9.01) (end 9 9.01) (width 0.6) (layer "B.Cu") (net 7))
 (segment (start 17.67 11.55) (end 18.61 12.49) (width 0.6) (layer "B.Cu") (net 8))
 (segment (start 9 11.55) (end 17.67 11.55) (width 0.6) (layer "B.Cu") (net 8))
 (segment (start 18.61 15.03) (end 11.4919 15.03) (width 0.6) (layer "B.Cu") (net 9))
 (segment (start 11.4919 15.03) (end 10.5519 14.09) (width 0.6) (layer "B.Cu") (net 9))
 (segment (start 9 14.09) (end 10.5519 14.09) (width 0.6) (layer "B.Cu") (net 9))
 (segment (start 9 16.629999) (end 17.67 16.629999) (width 0.6) (layer "B.Cu") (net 10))
 (segment (start 17.67 16.629999) (end 18.61 17.57) (width 0.6) (layer "B.Cu") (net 10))
 (segment (start 17.67 19.17) (end 18.61 20.11) (width 0.6) (layer "B.Cu") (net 11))
 (segment (start 9 19.17) (end 17.67 19.17) (width 0.6) (layer "B.Cu") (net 11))
 (segment (start 15.13 21.71) (end 18.61 25.19) (width 0.6) (layer "B.Cu") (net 12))
 (segment (start 9 21.71) (end 15.13 21.71) (width 0.6) (layer "B.Cu") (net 12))
 (segment (start 12.3 42.504) (end 12.3 44.3) (width 0.6) (layer "B.Cu") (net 20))
 (segment (start 15.7838 33.0962) (end 15.7838 39.0202) (width 0.6) (layer "B.Cu") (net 20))
 (segment (start 9.27 42.5562) (end 9.27 42.504) (width 0.6) (layer "B.Cu") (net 20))
 (segment (start 9.27 44.5) (end 9.27 44.3) (width 0.6) (layer "B.Cu") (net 20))
 (segment (start 9.27 42.504) (end 9.27 41) (width 0.6) (layer "B.Cu") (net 20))
 (segment (start 18.61 30.27) (end 15.7838 33.0962) (width 0.6) (layer "B.Cu") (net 20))
 (segment (start 9.27 42.6258) (end 9.27 42.5562) (width 0.6) (layer "B.Cu") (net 20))
 (segment (start 9.27 42.75) (end 9.27 42.6258) (width 0.6) (layer "B.Cu") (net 20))
 (segment (start 9.27 44.3) (end 9.27 42.75) (width 0.6) (layer "B.Cu") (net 20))
 (segment (start 12.3 42.504) (end 9.27 42.504) (width 0.6) (layer "B.Cu") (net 20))
 (segment (start 15.7838 39.0202) (end 12.3 42.504) (width 0.6) (layer "B.Cu") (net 20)))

